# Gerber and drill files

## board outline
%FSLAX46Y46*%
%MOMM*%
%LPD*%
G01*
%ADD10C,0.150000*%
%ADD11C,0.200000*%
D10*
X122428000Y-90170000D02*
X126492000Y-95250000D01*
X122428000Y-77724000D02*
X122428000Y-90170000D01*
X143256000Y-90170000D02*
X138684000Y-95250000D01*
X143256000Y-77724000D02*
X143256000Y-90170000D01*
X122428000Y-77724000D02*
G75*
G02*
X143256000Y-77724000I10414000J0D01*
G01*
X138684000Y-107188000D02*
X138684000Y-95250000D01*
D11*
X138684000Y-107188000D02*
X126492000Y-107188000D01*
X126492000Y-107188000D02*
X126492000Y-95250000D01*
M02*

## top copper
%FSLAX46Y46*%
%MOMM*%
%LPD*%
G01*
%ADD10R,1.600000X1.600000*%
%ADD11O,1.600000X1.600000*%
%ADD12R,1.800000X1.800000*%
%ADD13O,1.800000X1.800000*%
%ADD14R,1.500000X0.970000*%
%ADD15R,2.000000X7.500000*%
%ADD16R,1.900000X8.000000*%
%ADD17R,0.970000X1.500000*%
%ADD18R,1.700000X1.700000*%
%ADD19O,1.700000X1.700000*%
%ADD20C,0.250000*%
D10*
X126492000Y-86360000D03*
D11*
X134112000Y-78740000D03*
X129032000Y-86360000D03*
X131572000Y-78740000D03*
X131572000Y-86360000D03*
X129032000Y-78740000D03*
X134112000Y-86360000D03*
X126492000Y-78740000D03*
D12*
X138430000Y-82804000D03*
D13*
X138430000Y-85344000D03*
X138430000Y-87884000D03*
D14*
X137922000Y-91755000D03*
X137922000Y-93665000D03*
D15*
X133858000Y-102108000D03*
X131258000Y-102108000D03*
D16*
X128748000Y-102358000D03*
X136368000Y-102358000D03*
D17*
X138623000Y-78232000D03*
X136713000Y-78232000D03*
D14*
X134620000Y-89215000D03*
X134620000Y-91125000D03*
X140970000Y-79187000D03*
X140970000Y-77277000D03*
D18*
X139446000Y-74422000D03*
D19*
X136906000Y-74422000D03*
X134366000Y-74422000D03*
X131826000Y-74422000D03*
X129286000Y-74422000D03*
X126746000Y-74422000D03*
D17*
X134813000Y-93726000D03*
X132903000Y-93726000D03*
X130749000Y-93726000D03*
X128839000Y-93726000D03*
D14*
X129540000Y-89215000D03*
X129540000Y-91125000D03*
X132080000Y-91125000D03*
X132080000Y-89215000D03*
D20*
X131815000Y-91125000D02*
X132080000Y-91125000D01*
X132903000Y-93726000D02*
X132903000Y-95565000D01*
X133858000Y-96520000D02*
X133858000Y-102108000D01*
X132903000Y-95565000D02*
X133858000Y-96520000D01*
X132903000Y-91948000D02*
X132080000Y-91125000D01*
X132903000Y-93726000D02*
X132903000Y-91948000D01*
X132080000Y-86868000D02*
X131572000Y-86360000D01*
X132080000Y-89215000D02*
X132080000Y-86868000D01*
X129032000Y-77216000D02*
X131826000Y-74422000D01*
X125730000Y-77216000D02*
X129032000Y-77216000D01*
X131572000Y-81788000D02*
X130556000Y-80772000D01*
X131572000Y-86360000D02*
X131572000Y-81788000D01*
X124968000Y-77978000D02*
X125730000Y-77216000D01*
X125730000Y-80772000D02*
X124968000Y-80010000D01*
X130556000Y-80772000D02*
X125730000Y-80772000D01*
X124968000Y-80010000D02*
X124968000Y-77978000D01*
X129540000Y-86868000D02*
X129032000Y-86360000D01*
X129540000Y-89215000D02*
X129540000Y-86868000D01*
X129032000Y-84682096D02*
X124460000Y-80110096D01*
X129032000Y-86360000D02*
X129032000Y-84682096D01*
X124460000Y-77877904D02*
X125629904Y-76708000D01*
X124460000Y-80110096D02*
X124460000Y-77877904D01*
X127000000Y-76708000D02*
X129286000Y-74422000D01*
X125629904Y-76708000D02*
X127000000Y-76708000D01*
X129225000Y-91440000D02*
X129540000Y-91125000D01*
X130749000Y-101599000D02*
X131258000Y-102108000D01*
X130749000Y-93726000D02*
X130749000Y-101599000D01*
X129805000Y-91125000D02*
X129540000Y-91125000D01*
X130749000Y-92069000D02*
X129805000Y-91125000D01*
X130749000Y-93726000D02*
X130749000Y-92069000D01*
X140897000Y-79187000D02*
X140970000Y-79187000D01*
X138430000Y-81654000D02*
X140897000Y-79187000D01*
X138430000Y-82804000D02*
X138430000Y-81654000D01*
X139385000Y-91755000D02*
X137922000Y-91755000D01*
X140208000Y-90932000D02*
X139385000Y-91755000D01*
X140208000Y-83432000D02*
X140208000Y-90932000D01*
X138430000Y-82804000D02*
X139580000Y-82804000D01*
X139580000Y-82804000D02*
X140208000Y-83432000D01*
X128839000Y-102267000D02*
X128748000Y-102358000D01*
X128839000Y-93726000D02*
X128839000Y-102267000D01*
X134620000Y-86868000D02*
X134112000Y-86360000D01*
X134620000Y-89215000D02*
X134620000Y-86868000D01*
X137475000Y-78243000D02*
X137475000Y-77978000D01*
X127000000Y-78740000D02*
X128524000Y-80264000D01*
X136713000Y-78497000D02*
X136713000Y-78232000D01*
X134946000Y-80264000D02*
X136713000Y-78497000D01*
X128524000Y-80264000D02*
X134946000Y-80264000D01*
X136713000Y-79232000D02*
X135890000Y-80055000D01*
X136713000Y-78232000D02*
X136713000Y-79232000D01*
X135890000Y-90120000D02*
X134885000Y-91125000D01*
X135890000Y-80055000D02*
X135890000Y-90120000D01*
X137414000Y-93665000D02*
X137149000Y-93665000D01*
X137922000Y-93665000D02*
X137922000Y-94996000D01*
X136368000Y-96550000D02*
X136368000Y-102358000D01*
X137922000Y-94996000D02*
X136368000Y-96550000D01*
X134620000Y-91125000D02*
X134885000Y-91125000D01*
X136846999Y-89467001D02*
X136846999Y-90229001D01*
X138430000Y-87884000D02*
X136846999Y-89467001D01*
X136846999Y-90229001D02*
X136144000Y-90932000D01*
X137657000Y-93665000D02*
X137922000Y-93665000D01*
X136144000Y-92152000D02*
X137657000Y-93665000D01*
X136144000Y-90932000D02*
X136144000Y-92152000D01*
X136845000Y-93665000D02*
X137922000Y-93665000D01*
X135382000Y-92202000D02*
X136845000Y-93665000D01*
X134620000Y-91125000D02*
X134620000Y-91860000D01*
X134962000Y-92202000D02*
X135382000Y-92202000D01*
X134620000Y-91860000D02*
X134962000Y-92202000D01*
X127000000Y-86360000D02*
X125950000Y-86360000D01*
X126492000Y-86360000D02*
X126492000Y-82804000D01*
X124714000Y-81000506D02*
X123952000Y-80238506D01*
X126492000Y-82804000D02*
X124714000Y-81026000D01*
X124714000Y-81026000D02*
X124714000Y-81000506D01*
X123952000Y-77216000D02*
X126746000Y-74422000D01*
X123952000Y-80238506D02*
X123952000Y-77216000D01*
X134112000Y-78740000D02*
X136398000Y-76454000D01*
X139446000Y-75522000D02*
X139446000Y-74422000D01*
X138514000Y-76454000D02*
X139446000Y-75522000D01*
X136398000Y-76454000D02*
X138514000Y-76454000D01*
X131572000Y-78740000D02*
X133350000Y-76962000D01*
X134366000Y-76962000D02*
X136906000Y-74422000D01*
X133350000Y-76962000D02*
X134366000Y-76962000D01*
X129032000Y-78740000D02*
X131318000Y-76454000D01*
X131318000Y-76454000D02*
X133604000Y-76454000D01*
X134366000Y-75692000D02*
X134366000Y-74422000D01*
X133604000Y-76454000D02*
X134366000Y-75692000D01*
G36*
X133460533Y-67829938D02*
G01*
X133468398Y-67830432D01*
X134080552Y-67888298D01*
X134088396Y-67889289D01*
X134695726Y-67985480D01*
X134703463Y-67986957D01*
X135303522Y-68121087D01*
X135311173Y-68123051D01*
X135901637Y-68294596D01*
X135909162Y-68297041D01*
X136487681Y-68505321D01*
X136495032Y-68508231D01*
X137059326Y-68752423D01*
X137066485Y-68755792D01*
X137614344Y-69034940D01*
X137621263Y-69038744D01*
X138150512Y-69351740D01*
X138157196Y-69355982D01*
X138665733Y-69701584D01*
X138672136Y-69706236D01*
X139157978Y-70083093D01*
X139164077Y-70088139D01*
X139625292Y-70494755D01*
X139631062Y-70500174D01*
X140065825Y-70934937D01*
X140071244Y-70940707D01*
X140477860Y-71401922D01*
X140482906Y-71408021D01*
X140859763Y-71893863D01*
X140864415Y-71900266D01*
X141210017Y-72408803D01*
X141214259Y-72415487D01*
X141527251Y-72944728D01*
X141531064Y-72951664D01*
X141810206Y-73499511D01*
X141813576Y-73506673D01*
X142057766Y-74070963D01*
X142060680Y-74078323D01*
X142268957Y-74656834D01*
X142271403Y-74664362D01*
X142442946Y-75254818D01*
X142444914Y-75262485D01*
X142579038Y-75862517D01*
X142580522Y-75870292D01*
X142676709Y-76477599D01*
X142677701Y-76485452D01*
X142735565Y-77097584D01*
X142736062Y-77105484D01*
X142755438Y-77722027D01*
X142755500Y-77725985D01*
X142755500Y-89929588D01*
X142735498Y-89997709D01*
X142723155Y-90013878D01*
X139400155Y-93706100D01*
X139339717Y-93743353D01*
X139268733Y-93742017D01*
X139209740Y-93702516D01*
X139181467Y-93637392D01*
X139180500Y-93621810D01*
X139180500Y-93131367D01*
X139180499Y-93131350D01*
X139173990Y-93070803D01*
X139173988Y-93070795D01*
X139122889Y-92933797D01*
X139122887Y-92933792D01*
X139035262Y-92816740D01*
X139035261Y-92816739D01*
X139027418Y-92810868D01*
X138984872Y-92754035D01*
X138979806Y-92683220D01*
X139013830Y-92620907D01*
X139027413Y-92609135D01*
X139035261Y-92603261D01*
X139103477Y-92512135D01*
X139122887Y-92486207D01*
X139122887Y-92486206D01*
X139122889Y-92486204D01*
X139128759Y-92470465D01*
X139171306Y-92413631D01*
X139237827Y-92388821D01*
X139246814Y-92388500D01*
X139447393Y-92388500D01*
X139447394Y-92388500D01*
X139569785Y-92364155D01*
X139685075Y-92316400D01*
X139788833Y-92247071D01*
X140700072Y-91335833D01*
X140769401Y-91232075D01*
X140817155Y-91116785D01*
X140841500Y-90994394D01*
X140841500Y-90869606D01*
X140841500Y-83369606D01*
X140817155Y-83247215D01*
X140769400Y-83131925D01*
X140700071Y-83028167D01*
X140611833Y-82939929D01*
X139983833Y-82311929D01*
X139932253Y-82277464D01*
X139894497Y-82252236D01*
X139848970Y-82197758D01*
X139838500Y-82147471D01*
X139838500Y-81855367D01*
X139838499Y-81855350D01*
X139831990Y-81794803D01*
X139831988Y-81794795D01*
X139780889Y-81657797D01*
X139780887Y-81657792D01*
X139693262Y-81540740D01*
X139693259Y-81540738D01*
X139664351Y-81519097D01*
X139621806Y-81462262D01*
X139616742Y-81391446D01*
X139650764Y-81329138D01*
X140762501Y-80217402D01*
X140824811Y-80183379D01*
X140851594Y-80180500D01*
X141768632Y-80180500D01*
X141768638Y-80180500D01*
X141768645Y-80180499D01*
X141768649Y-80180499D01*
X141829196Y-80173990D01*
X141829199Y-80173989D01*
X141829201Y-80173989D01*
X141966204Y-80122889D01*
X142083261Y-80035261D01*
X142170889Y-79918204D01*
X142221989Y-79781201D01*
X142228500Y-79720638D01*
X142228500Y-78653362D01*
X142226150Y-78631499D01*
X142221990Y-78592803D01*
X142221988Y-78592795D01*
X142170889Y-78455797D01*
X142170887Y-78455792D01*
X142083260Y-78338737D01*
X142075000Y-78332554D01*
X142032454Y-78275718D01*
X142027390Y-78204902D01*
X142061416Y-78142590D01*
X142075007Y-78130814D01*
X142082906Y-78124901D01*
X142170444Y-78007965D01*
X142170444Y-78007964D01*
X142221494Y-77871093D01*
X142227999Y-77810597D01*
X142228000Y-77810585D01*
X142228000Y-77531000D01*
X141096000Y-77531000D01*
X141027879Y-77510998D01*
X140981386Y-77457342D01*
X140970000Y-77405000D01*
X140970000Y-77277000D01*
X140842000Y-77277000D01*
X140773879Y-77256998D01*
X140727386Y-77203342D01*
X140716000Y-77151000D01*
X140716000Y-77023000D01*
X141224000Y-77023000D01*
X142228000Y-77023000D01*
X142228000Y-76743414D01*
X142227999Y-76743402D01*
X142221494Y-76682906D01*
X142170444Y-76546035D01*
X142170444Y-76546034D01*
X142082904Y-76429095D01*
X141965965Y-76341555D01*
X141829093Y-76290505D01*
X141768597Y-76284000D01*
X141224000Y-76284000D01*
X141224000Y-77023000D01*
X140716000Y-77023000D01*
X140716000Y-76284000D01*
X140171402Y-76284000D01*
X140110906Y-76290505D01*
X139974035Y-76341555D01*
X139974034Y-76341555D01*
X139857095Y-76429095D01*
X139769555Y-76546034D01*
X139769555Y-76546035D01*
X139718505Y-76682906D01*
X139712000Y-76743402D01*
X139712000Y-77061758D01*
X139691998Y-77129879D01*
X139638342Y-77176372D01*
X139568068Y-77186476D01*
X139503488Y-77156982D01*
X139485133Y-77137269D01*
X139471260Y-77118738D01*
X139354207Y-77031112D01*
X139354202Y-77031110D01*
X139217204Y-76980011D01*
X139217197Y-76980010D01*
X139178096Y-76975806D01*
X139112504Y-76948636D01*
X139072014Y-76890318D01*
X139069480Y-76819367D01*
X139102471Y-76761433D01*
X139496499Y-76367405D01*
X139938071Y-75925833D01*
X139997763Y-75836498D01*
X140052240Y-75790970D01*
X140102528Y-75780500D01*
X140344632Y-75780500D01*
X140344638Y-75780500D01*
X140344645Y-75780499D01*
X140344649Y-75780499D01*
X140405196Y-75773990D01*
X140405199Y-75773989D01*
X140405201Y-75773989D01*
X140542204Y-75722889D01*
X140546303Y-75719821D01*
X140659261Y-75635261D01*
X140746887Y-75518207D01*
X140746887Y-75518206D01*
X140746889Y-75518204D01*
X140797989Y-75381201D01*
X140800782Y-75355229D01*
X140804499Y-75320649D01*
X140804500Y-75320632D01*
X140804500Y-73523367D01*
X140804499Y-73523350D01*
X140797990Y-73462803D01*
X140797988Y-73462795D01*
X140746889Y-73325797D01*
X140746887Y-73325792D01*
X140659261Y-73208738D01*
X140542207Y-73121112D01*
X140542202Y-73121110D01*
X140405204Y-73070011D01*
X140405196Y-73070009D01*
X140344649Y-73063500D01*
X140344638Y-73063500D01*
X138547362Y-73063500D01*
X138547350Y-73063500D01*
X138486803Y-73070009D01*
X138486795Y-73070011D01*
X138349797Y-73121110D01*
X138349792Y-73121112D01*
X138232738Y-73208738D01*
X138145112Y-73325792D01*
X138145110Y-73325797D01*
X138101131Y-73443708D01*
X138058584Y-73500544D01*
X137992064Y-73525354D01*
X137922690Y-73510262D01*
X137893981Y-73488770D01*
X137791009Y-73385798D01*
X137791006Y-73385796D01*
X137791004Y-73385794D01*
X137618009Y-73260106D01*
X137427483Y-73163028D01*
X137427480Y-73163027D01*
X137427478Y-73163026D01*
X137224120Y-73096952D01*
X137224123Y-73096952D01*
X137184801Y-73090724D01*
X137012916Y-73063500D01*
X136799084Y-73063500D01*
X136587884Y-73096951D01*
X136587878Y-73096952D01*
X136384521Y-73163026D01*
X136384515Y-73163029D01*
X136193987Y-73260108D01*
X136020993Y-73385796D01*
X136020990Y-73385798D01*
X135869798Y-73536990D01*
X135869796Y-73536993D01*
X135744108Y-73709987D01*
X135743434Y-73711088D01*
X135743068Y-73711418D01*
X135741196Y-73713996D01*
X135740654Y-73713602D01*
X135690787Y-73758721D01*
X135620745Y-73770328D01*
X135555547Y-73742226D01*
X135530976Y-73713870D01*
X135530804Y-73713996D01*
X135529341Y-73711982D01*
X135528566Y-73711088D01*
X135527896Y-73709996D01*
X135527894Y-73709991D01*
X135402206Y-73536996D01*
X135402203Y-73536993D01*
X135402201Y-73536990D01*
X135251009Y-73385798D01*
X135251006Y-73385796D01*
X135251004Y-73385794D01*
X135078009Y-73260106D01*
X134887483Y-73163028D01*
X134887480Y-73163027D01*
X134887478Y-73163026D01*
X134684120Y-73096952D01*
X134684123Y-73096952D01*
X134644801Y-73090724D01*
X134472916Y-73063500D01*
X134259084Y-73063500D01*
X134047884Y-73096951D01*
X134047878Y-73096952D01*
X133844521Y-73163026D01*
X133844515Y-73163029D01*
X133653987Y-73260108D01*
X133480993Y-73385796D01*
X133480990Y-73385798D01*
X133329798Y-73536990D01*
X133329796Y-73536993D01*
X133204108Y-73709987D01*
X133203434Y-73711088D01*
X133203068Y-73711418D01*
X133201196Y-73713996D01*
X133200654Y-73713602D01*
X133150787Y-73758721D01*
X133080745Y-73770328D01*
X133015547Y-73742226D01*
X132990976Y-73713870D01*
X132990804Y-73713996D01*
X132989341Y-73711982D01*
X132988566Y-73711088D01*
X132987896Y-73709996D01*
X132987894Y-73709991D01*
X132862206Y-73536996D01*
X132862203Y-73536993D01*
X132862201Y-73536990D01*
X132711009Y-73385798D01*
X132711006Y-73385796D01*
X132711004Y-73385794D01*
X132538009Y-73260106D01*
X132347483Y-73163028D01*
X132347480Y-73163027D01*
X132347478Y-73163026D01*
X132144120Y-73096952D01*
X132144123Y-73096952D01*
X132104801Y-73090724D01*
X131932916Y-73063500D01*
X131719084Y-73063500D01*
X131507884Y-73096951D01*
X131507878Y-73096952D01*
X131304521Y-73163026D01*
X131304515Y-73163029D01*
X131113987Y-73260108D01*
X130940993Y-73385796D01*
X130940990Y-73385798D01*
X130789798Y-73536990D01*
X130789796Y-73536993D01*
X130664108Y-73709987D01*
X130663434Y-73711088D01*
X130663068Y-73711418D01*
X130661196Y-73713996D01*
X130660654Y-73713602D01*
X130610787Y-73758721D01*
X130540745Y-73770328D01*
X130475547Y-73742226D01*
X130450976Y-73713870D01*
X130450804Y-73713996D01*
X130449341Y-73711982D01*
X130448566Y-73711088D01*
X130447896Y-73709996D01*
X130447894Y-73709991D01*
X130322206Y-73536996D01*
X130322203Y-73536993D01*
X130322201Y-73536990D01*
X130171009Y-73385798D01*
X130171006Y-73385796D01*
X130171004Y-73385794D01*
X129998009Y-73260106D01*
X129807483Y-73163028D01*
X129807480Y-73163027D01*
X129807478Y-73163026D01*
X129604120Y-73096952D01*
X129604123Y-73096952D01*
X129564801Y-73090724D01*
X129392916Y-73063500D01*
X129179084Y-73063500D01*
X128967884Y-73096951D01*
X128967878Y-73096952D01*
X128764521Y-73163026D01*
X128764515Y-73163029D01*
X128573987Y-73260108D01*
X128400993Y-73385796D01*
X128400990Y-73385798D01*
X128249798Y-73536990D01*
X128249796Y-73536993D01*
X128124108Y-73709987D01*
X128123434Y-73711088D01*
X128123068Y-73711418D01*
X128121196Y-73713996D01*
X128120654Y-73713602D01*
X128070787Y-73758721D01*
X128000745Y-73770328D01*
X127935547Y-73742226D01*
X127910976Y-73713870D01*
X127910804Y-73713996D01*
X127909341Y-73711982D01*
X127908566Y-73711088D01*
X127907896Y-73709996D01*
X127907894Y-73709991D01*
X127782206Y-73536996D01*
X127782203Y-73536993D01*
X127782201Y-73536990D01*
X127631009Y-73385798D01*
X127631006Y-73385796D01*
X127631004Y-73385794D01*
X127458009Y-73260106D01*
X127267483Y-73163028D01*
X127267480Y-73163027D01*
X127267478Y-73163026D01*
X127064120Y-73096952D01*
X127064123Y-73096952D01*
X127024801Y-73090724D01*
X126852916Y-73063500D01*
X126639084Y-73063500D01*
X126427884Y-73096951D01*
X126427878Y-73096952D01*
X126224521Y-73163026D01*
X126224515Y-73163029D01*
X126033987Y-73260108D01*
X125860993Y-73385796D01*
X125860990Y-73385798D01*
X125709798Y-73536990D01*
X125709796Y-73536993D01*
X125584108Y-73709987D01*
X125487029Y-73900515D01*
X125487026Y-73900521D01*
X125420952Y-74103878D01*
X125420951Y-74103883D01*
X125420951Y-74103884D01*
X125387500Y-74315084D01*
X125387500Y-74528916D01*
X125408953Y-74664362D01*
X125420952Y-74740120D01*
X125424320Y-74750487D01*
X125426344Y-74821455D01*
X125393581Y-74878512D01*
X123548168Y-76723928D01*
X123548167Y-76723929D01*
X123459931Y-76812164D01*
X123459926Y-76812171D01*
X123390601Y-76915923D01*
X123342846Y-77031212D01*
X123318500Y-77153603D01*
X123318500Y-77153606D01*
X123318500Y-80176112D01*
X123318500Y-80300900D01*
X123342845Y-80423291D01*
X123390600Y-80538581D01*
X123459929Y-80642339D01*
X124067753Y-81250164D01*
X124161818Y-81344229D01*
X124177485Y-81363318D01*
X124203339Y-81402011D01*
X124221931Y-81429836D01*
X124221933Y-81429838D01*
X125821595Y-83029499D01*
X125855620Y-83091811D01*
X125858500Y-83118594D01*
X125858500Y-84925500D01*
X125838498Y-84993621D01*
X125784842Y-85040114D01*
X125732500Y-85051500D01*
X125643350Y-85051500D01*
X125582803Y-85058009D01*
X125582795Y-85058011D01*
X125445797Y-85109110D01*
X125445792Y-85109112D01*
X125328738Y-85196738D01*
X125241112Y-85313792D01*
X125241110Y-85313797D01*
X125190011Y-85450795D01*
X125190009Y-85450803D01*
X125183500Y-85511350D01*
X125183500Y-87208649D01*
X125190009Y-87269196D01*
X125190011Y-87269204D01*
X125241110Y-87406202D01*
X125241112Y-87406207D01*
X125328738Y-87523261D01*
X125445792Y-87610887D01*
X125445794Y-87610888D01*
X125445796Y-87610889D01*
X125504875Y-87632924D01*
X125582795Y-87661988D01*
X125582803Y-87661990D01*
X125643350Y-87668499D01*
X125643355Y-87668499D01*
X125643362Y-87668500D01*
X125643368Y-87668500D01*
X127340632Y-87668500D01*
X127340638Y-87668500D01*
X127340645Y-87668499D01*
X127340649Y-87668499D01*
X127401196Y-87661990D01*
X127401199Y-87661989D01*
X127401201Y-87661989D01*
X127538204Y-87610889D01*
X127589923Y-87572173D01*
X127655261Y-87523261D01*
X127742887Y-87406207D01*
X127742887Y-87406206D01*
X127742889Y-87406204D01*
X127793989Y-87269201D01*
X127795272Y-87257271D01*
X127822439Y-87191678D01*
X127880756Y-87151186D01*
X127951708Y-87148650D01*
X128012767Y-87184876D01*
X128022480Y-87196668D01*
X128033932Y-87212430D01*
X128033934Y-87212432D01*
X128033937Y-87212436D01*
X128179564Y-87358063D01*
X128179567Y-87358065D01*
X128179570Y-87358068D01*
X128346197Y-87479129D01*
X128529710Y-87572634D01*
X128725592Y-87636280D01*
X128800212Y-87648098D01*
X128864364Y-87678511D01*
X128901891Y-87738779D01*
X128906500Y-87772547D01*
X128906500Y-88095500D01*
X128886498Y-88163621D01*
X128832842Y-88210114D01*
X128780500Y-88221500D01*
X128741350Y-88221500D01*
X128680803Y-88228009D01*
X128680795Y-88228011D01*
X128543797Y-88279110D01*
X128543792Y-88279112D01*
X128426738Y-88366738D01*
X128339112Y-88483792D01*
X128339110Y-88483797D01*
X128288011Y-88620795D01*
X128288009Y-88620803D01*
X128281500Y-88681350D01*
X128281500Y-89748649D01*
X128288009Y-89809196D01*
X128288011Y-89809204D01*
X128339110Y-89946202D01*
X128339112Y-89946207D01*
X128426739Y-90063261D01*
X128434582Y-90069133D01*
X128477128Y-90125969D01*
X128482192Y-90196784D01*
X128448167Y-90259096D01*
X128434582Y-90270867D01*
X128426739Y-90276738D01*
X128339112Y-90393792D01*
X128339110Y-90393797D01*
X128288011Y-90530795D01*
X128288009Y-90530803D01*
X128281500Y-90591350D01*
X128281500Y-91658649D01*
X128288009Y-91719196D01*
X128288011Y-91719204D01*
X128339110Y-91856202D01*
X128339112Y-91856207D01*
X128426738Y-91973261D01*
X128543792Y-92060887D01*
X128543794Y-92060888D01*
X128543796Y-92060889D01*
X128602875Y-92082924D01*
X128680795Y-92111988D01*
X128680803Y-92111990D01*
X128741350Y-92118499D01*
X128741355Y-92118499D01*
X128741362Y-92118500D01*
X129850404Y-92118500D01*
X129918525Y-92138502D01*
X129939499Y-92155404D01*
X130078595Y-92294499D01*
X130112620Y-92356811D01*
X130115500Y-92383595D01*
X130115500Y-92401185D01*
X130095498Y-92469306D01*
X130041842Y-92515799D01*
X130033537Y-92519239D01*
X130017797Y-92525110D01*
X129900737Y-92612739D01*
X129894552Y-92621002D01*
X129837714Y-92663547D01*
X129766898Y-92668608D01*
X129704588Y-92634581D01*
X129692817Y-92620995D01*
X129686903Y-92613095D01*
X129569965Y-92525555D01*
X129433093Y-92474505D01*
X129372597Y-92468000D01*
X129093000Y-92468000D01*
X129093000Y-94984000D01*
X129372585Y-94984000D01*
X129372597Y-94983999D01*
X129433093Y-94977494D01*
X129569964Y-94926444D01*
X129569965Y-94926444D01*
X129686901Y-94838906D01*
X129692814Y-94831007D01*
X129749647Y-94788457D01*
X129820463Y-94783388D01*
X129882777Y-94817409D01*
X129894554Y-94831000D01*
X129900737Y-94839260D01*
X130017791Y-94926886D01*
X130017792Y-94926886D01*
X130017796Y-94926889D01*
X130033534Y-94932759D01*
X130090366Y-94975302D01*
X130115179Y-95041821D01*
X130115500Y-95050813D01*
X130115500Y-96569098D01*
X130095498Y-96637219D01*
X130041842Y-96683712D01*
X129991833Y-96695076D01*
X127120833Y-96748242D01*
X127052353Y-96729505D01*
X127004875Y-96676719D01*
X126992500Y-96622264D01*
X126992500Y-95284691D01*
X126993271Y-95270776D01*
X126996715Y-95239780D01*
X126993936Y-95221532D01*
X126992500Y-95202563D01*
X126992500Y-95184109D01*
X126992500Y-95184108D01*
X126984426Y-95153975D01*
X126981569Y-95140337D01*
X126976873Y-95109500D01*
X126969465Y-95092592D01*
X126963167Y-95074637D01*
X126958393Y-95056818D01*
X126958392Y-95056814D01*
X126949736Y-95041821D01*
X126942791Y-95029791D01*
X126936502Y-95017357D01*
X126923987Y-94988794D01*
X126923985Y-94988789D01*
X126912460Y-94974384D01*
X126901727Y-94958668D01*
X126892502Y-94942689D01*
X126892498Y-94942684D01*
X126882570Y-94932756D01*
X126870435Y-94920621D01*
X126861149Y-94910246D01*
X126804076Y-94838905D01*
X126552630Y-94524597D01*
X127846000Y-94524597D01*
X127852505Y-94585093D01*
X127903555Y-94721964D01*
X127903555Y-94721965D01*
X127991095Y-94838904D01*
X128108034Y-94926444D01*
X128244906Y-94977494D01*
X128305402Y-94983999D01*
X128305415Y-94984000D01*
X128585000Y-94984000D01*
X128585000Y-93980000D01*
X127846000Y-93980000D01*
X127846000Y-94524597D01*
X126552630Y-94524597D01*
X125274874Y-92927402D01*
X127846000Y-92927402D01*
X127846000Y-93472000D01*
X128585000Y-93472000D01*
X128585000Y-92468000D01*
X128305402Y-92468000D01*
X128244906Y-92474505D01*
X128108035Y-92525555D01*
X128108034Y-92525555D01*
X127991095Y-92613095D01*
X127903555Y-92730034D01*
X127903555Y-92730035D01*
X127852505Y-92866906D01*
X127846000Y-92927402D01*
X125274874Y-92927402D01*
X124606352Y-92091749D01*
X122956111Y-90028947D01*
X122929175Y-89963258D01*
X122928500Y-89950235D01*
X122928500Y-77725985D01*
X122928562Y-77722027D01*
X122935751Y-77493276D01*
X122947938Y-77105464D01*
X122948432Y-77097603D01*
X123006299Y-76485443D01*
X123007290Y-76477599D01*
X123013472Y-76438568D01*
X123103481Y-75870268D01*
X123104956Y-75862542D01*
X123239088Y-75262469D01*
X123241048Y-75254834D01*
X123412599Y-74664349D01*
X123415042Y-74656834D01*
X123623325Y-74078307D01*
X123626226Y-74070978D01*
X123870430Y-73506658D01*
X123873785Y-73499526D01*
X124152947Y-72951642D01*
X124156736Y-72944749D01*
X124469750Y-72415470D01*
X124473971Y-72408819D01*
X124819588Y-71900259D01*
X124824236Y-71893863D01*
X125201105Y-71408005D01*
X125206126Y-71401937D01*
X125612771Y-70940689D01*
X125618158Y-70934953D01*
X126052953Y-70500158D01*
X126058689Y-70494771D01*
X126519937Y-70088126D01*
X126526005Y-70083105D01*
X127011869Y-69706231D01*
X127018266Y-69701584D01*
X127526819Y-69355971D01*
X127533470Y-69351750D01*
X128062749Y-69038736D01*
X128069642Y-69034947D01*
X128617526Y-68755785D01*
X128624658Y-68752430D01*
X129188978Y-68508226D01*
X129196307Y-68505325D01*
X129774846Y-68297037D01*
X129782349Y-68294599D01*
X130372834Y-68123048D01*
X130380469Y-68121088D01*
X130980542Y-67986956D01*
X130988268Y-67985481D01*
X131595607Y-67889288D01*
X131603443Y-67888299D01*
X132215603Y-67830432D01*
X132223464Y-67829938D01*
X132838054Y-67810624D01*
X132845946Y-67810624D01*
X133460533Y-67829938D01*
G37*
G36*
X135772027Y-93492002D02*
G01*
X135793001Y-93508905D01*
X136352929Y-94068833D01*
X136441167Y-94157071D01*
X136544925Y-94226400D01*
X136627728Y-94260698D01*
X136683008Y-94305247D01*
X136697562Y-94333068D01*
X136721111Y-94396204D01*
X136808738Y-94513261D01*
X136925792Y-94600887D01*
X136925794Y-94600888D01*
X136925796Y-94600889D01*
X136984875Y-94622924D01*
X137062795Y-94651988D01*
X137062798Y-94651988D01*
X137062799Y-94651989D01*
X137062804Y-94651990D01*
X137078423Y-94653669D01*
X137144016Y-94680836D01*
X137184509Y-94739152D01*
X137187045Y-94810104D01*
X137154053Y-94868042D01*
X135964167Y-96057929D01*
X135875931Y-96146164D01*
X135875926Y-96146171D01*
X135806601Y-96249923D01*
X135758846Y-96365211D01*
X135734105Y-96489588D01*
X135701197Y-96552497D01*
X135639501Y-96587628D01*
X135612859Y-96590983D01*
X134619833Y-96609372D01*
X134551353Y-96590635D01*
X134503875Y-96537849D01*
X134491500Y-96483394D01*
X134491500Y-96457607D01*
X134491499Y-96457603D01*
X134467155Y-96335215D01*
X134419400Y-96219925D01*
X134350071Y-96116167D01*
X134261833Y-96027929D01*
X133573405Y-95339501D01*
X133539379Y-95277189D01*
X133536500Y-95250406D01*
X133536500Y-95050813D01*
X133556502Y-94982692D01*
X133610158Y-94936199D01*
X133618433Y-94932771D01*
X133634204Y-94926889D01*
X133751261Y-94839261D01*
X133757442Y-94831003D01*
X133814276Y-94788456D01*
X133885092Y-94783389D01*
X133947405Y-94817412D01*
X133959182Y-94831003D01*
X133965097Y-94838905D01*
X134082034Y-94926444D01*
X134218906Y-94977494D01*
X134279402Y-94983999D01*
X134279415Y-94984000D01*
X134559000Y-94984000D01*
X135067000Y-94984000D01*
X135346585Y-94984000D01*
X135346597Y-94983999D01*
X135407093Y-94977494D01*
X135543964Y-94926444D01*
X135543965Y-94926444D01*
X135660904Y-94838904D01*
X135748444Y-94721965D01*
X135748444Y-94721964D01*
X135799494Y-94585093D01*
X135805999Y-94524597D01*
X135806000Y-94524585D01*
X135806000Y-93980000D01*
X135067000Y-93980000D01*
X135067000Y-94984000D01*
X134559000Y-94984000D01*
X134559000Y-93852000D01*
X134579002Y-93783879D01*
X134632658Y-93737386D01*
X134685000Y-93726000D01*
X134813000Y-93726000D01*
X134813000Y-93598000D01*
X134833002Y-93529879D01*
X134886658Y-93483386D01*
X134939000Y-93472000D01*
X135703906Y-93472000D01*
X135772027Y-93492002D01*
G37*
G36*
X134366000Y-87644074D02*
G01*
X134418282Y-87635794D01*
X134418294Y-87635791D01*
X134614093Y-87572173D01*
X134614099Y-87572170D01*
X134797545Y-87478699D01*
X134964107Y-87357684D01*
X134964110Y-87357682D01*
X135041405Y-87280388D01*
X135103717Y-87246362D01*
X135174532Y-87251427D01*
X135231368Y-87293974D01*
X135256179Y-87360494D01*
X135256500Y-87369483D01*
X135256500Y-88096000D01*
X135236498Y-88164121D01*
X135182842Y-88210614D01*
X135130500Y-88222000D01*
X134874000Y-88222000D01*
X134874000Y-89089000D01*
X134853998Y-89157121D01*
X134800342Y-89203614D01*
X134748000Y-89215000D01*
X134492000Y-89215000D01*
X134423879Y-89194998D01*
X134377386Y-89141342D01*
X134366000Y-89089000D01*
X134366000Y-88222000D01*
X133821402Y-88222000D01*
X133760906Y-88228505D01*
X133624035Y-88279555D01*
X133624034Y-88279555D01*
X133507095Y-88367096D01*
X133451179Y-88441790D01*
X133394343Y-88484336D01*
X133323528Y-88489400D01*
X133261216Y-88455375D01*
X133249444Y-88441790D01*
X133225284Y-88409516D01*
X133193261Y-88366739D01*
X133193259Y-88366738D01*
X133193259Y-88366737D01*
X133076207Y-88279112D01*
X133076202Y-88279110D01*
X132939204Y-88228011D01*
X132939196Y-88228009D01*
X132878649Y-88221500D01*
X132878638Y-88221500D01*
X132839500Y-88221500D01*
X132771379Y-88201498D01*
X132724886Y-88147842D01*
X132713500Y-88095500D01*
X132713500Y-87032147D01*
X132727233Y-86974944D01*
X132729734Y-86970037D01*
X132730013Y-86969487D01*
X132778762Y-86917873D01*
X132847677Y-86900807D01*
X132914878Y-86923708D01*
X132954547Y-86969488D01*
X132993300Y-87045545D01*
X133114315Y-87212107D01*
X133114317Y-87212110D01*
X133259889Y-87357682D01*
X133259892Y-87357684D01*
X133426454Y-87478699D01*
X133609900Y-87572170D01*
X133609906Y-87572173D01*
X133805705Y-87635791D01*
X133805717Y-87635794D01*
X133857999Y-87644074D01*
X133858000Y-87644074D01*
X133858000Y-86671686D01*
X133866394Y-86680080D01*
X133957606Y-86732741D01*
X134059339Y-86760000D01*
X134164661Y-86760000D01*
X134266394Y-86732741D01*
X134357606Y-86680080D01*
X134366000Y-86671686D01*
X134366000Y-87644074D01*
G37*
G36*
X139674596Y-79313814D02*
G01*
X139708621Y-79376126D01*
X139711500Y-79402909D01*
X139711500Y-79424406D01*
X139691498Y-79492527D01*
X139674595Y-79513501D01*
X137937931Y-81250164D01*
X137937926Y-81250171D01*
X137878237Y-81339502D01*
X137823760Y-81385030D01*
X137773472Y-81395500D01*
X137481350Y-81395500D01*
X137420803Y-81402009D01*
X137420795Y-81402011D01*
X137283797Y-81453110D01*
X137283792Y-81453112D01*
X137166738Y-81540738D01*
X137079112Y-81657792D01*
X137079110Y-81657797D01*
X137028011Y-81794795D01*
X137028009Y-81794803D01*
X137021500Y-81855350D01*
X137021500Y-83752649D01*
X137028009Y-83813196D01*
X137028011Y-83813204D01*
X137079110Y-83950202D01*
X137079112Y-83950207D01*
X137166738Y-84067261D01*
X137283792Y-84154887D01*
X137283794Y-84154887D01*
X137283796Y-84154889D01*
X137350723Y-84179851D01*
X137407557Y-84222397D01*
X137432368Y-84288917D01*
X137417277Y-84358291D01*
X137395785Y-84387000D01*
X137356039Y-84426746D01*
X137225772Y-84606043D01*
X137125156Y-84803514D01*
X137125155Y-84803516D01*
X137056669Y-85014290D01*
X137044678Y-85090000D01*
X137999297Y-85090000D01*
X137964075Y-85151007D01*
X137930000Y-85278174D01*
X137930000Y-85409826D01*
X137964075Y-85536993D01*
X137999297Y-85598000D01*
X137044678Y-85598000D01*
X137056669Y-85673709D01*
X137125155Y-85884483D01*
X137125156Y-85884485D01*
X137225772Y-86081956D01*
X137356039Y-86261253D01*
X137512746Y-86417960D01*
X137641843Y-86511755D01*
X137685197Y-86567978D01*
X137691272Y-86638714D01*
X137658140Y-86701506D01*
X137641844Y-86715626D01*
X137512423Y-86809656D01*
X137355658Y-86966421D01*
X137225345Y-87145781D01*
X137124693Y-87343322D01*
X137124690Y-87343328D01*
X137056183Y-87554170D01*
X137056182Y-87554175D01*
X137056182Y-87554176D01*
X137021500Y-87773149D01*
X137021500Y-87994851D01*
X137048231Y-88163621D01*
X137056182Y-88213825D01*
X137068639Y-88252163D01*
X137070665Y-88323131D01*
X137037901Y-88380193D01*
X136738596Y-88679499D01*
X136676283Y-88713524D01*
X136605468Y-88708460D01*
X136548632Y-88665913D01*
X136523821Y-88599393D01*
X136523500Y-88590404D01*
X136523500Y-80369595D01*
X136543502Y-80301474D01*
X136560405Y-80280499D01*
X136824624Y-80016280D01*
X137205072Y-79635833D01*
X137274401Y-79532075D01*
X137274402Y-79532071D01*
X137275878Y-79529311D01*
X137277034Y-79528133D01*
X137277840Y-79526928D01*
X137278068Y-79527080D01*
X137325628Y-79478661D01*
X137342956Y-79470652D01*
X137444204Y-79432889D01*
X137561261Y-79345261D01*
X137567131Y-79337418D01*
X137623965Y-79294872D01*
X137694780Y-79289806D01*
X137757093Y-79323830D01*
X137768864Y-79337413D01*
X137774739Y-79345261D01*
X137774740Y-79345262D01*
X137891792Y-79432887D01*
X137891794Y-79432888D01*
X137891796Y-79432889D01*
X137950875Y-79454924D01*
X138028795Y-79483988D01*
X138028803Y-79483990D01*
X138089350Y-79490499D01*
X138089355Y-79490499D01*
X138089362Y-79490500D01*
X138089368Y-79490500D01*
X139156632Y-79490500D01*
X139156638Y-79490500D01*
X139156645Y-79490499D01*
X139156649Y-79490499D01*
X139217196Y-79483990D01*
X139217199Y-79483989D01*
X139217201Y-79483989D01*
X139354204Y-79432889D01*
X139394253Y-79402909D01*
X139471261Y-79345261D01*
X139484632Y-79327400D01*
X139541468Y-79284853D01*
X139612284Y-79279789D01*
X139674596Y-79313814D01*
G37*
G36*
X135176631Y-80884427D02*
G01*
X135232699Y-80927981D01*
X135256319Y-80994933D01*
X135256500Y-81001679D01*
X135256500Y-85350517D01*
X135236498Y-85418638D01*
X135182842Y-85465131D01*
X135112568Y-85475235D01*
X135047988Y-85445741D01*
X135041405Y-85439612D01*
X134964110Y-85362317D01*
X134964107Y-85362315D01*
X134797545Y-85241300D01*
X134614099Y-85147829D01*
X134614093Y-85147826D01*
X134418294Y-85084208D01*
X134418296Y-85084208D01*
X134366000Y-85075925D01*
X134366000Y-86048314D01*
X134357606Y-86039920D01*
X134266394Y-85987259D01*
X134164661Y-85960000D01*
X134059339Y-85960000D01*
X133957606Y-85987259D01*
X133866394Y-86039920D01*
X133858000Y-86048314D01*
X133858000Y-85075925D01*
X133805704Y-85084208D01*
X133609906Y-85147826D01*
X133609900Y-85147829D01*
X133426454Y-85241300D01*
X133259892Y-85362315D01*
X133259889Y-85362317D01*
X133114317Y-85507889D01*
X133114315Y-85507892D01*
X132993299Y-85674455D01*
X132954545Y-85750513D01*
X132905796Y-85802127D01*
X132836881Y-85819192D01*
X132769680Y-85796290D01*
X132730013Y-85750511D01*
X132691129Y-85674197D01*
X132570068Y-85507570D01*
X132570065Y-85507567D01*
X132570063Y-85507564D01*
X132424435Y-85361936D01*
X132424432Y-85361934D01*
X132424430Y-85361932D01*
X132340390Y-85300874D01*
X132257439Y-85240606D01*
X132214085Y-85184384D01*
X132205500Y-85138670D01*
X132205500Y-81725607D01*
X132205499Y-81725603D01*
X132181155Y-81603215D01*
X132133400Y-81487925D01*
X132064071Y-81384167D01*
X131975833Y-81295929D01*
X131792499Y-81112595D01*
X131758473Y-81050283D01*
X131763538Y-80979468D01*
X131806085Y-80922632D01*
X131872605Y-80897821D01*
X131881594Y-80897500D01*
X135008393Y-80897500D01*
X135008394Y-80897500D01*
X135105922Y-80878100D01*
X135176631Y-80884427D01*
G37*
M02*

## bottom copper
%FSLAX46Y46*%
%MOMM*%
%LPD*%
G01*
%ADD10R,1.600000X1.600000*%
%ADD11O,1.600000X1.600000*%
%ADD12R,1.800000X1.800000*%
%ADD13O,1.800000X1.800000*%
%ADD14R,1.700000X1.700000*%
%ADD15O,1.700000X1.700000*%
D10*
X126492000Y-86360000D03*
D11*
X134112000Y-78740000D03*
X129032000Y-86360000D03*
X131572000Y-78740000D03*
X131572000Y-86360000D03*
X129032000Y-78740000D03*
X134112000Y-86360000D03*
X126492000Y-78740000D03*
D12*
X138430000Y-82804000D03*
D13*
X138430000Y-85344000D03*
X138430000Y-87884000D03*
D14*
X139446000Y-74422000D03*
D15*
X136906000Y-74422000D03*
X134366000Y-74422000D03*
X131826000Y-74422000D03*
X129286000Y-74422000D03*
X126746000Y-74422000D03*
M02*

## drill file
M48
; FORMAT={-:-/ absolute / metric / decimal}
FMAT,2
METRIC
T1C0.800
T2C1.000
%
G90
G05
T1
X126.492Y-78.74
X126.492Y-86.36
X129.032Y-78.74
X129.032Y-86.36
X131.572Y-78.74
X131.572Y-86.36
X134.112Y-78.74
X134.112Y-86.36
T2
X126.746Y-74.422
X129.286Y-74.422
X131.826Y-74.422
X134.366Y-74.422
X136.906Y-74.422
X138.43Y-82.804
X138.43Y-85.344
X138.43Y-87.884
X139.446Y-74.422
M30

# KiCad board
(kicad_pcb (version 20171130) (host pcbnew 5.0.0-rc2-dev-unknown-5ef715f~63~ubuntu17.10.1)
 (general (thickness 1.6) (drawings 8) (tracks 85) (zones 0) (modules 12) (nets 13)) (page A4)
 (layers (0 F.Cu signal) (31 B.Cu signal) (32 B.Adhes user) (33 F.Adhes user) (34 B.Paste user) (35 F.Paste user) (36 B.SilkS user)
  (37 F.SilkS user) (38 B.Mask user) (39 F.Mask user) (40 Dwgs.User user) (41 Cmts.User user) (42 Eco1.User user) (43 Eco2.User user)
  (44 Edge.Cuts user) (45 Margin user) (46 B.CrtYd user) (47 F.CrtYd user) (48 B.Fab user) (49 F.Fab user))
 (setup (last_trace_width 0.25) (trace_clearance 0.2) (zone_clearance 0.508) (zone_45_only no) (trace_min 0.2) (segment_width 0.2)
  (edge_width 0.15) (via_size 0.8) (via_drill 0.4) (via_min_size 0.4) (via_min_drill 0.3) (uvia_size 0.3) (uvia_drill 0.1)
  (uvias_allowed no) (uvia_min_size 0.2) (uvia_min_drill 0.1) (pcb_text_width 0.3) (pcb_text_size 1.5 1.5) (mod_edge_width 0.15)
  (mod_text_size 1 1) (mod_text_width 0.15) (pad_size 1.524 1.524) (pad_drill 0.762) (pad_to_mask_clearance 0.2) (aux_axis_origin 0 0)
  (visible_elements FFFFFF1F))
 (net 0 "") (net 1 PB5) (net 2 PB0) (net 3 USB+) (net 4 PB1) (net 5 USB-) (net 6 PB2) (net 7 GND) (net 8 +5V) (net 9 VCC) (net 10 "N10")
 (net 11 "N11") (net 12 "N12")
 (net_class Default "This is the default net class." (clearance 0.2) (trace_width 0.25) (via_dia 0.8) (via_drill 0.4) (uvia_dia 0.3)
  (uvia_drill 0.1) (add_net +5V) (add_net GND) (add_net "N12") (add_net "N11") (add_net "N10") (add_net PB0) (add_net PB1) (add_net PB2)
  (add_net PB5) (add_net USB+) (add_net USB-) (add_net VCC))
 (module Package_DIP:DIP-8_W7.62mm (layer F.Cu) (at 126.492 86.36 90)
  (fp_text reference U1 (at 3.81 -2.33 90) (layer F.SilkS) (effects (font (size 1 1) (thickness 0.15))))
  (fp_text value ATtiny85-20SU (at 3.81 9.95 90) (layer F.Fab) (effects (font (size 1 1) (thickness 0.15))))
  (pad 1 thru_hole rect (at 0 0 90) (size 1.6 1.6) (drill 0.8) (layers *.Cu *.Mask) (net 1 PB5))
  (pad 5 thru_hole oval (at 7.62 7.62 90) (size 1.6 1.6) (drill 0.8) (layers *.Cu *.Mask) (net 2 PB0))
  (pad 2 thru_hole oval (at 0 2.54 90) (size 1.6 1.6) (drill 0.8) (layers *.Cu *.Mask) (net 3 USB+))
  (pad 6 thru_hole oval (at 7.62 5.08 90) (size 1.6 1.6) (drill 0.8) (layers *.Cu *.Mask) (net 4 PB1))
  (pad 3 thru_hole oval (at 0 5.08 90) (size 1.6 1.6) (drill 0.8) (layers *.Cu *.Mask) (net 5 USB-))
  (pad 7 thru_hole oval (at 7.62 2.54 90) (size 1.6 1.6) (drill 0.8) (layers *.Cu *.Mask) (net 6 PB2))
  (pad 4 thru_hole oval (at 0 7.62 90) (size 1.6 1.6) (drill 0.8) (layers *.Cu *.Mask) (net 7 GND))
  (pad 8 thru_hole oval (at 7.62 0 90) (size 1.6 1.6) (drill 0.8) (layers *.Cu *.Mask) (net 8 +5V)))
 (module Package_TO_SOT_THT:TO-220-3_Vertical (layer F.Cu) (at 138.43 82.804 270)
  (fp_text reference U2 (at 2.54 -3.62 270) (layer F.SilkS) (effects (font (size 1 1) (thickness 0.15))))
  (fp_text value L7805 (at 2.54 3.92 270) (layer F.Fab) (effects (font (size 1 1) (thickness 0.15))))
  (pad 1 thru_hole rect (at 0 0 270) (size 1.8 1.8) (drill 1) (layers *.Cu *.Mask) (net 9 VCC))
  (pad 2 thru_hole oval (at 2.54 0 270) (size 1.8 1.8) (drill 1) (layers *.Cu *.Mask) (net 7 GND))
  (pad 3 thru_hole oval (at 5.08 0 270) (size 1.8 1.8) (drill 1) (layers *.Cu *.Mask) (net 8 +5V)))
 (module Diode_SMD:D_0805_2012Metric (layer F.Cu) (at 137.922 92.71 270)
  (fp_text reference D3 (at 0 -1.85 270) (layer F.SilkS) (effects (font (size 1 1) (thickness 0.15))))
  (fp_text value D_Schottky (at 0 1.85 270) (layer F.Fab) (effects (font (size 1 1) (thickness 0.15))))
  (pad 1 smd rect (at -0.955 0 270) (size 0.97 1.5) (layers F.Cu F.Paste F.Mask) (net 9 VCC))
  (pad 2 smd rect (at 0.955 0 270) (size 0.97 1.5) (layers F.Cu F.Paste F.Mask) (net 8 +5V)))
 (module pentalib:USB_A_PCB (layer F.Cu) (at 132.558 107.258)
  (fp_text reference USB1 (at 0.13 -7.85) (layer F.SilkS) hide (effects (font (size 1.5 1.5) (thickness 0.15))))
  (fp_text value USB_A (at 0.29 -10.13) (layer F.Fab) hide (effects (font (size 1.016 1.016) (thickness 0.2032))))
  (pad 2 connect rect (at 1.3 -5.15) (size 2 7.5) (layers F.Cu F.Mask) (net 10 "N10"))
  (pad 3 connect rect (at -1.3 -5.15) (size 2 7.5) (layers F.Cu F.Mask) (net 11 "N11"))
  (pad 4 connect rect (at -3.81 -4.9) (size 1.9 8) (layers F.Cu F.Mask) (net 7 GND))
  (pad 1 connect rect (at 3.81 -4.9) (size 1.9 8) (layers F.Cu F.Mask) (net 8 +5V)))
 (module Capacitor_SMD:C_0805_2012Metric (layer F.Cu) (at 137.668 78.232 180)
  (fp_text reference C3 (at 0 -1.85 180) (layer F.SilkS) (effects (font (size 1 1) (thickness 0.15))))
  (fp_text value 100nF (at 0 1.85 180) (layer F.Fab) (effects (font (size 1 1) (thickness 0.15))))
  (pad 1 smd rect (at -0.955 0 180) (size 0.97 1.5) (layers F.Cu F.Paste F.Mask) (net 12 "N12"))
  (pad 2 smd rect (at 0.955 0 180) (size 0.97 1.5) (layers F.Cu F.Paste F.Mask) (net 8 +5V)))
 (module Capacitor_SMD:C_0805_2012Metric (layer F.Cu) (at 134.62 90.17 90)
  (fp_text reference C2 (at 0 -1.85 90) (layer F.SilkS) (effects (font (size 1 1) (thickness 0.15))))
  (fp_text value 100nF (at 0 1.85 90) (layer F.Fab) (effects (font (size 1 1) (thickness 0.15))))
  (pad 2 smd rect (at 0.955 0 90) (size 0.97 1.5) (layers F.Cu F.Paste F.Mask) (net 7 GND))
  (pad 1 smd rect (at -0.955 0 90) (size 0.97 1.5) (layers F.Cu F.Paste F.Mask) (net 8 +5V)))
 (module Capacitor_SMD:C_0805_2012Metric (layer F.Cu) (at 140.97 78.232 90)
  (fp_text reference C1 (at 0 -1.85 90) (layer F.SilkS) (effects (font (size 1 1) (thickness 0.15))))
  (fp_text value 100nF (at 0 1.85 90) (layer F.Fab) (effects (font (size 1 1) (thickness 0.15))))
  (pad 1 smd rect (at -0.955 0 90) (size 0.97 1.5) (layers F.Cu F.Paste F.Mask) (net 9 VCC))
  (pad 2 smd rect (at 0.955 0 90) (size 0.97 1.5) (layers F.Cu F.Paste F.Mask) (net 7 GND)))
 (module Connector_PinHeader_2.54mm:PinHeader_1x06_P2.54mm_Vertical (layer F.Cu) (at 139.446 74.422 270)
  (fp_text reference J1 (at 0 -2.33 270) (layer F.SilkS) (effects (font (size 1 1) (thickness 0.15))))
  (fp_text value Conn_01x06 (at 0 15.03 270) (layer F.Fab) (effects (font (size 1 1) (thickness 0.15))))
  (pad 1 thru_hole rect (at 0 0 270) (size 1.7 1.7) (drill 1) (layers *.Cu *.Mask) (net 2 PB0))
  (pad 2 thru_hole oval (at 0 2.54 270) (size 1.7 1.7) (drill 1) (layers *.Cu *.Mask) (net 4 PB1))
  (pad 3 thru_hole oval (at 0 5.08 270) (size 1.7 1.7) (drill 1) (layers *.Cu *.Mask) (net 6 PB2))
  (pad 4 thru_hole oval (at 0 7.62 270) (size 1.7 1.7) (drill 1) (layers *.Cu *.Mask) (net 5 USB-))
  (pad 5 thru_hole oval (at 0 10.16 270) (size 1.7 1.7) (drill 1) (layers *.Cu *.Mask) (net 3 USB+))
  (pad 6 thru_hole oval (at 0 12.7 270) (size 1.7 1.7) (drill 1) (layers *.Cu *.Mask) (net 1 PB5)))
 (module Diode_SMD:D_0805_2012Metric (layer F.Cu) (at 133.858 93.726)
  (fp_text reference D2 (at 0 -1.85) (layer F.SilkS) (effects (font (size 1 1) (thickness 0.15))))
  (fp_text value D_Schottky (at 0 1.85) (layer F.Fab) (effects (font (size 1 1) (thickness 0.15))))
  (pad 2 smd rect (at 0.955 0) (size 0.97 1.5) (layers F.Cu F.Paste F.Mask) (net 7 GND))
  (pad 1 smd rect (at -0.955 0) (size 0.97 1.5) (layers F.Cu F.Paste F.Mask) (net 10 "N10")))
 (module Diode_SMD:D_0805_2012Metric (layer F.Cu) (at 129.794 93.726 180)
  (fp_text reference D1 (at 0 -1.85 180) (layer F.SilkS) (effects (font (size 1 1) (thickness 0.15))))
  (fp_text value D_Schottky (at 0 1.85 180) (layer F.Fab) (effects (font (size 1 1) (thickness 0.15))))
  (pad 1 smd rect (at -0.955 0 180) (size 0.97 1.5) (layers F.Cu F.Paste F.Mask) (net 11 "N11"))
  (pad 2 smd rect (at 0.955 0 180) (size 0.97 1.5) (layers F.Cu F.Paste F.Mask) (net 7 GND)))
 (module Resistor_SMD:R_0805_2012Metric (layer F.Cu) (at 129.54 90.17 90)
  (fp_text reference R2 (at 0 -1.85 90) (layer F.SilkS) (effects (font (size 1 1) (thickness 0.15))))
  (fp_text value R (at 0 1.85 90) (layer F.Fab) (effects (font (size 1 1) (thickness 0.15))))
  (pad 2 smd rect (at 0.955 0 90) (size 0.97 1.5) (layers F.Cu F.Paste F.Mask) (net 3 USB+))
  (pad 1 smd rect (at -0.955 0 90) (size 0.97 1.5) (layers F.Cu F.Paste F.Mask) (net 11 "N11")))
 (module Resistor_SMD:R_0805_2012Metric (layer F.Cu) (at 132.08 90.17 90)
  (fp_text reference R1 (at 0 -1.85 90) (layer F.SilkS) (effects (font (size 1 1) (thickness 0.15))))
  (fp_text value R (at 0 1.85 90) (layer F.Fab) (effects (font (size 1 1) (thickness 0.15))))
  (pad 1 smd rect (at -0.955 0 90) (size 0.97 1.5) (layers F.Cu F.Paste F.Mask) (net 10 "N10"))
  (pad 2 smd rect (at 0.955 0 90) (size 0.97 1.5) (layers F.Cu F.Paste F.Mask) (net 5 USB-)))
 (gr_line (start 122.428 90.17) (end 126.492 95.25) (layer Edge.Cuts) (width 0.15))
 (gr_line (start 122.428 77.724) (end 122.428 90.17) (layer Edge.Cuts) (width 0.15))
 (gr_line (start 143.256 90.17) (end 138.684 95.25) (layer Edge.Cuts) (width 0.15))
 (gr_line (start 143.256 77.724) (end 143.256 90.17) (layer Edge.Cuts) (width 0.15))
 (gr_arc (start 132.842 77.724) (end 143.256 77.724) (angle -180) (layer Edge.Cuts) (width 0.15))
 (gr_line (start 138.684 107.188) (end 138.684 95.25) (layer Edge.Cuts) (width 0.15))
 (gr_line (start 138.684 107.188) (end 126.492 107.188) (layer Edge.Cuts) (width 0.2))
 (gr_line (start 126.492 107.188) (end 126.492 95.25) (layer Edge.Cuts) (width 0.2))
 (segment (start 131.815 91.125) (end 132.08 91.125) (width 0.25) (layer F.Cu) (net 10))
 (segment (start 132.903 93.726) (end 132.903 95.565) (width 0.25) (layer F.Cu) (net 10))
 (segment (start 133.858 96.52) (end 133.858 102.108) (width 0.25) (layer F.Cu) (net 10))
 (segment (start 132.903 95.565) (end 133.858 96.52) (width 0.25) (layer F.Cu) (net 10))
 (segment (start 132.903 91.948) (end 132.08 91.125) (width 0.25) (layer F.Cu) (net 10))
 (segment (start 132.903 93.726) (end 132.903 91.948) (width 0.25) (layer F.Cu) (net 10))
 (segment (start 132.08 86.868) (end 131.572 86.36) (width 0.25) (layer F.Cu) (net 5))
 (segment (start 132.08 89.215) (end 132.08 86.868) (width 0.25) (layer F.Cu) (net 5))
 (segment (start 129.032 77.216) (end 131.826 74.422) (width 0.25) (layer F.Cu) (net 5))
 (segment (start 125.73 77.216) (end 129.032 77.216) (width 0.25) (layer F.Cu) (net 5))
 (segment (start 131.572 81.788) (end 130.556 80.772) (width 0.25) (layer F.Cu) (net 5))
 (segment (start 131.572 86.36) (end 131.572 81.788) (width 0.25) (layer F.Cu) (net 5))
 (segment (start 124.968 77.978) (end 125.73 77.216) (width 0.25) (layer F.Cu) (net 5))
 (segment (start 125.73 80.772) (end 124.968 80.01) (width 0.25) (layer F.Cu) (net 5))
 (segment (start 130.556 80.772) (end 125.73 80.772) (width 0.25) (layer F.Cu) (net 5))
 (segment (start 124.968 80.01) (end 124.968 77.978) (width 0.25) (layer F.Cu) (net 5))
 (segment (start 129.54 86.868) (end 129.032 86.36) (width 0.25) (layer F.Cu) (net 3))
 (segment (start 129.54 89.215) (end 129.54 86.868) (width 0.25) (layer F.Cu) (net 3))
 (segment (start 129.032 84.682096) (end 124.46 80.110096) (width 0.25) (layer F.Cu) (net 3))
 (segment (start 129.032 86.36) (end 129.032 84.682096) (width 0.25) (layer F.Cu) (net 3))
 (segment (start 124.46 77.877904) (end 125.629904 76.708) (width 0.25) (layer F.Cu) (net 3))
 (segment (start 124.46 80.110096) (end 124.46 77.877904) (width 0.25) (layer F.Cu) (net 3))
 (segment (start 127 76.708) (end 129.286 74.422) (width 0.25) (layer F.Cu) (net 3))
 (segment (start 125.629904 76.708) (end 127 76.708) (width 0.25) (layer F.Cu) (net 3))
 (segment (start 129.225 91.44) (end 129.54 91.125) (width 0.25) (layer F.Cu) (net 11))
 (segment (start 130.749 101.599) (end 131.258 102.108) (width 0.25) (layer F.Cu) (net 11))
 (segment (start 130.749 93.726) (end 130.749 101.599) (width 0.25) (layer F.Cu) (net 11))
 (segment (start 129.805 91.125) (end 129.54 91.125) (width 0.25) (layer F.Cu) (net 11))
 (segment (start 130.749 92.069) (end 129.805 91.125) (width 0.25) (layer F.Cu) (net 11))
 (segment (start 130.749 93.726) (end 130.749 92.069) (width 0.25) (layer F.Cu) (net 11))
 (segment (start 140.897 79.187) (end 140.97 79.187) (width 0.25) (layer F.Cu) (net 9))
 (segment (start 138.43 81.654) (end 140.897 79.187) (width 0.25) (layer F.Cu) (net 9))
 (segment (start 138.43 82.804) (end 138.43 81.654) (width 0.25) (layer F.Cu) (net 9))
 (segment (start 139.385 91.755) (end 137.922 91.755) (width 0.25) (layer F.Cu) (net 9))
 (segment (start 140.208 90.932) (end 139.385 91.755) (width 0.25) (layer F.Cu) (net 9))
 (segment (start 140.208 83.432) (end 140.208 90.932) (width 0.25) (layer F.Cu) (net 9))
 (segment (start 138.43 82.804) (end 139.58 82.804) (width 0.25) (layer F.Cu) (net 9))
 (segment (start 139.58 82.804) (end 140.208 83.432) (width 0.25) (layer F.Cu) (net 9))
 (segment (start 128.839 102.267) (end 128.748 102.358) (width 0.25) (layer F.Cu) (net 7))
 (segment (start 128.839 93.726) (end 128.839 102.267) (width 0.25) (layer F.Cu) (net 7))
 (segment (start 134.62 86.868) (end 134.112 86.36) (width 0.25) (layer F.Cu) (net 7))
 (segment (start 134.62 89.215) (end 134.62 86.868) (width 0.25) (layer F.Cu) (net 7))
 (segment (start 137.475 78.243) (end 137.475 77.978) (width 0.25) (layer F.Cu) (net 8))
 (segment (start 127 78.74) (end 128.524 80.264) (width 0.25) (layer F.Cu) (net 8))
 (segment (start 136.713 78.497) (end 136.713 78.232) (width 0.25) (layer F.Cu) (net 8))
 (segment (start 134.946 80.264) (end 136.713 78.497) (width 0.25) (layer F.Cu) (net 8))
 (segment (start 128.524 80.264) (end 134.946 80.264) (width 0.25) (layer F.Cu) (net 8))
 (segment (start 136.713 79.232) (end 135.89 80.055) (width 0.25) (layer F.Cu) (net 8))
 (segment (start 136.713 78.232) (end 136.713 79.232) (width 0.25) (layer F.Cu) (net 8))
 (segment (start 135.89 90.12) (end 134.885 91.125) (width 0.25) (layer F.Cu) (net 8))
 (segment (start 135.89 80.055) (end 135.89 90.12) (width 0.25) (layer F.Cu) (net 8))
 (segment (start 137.414 93.665) (end 137.149 93.665) (width 0.25) (layer F.Cu) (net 8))
 (segment (start 137.922 93.665) (end 137.922 94.996) (width 0.25) (layer F.Cu) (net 8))
 (segment (start 136.368 96.55) (end 136.368 102.358) (width 0.25) (layer F.Cu) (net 8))
 (segment (start 137.922 94.996) (end 136.368 96.55) (width 0.25) (layer F.Cu) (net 8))
 (segment (start 134.62 91.125) (end 134.885 91.125) (width 0.25) (layer F.Cu) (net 8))
 (segment (start 136.846999 89.467001) (end 136.846999 90.229001) (width 0.25) (layer F.Cu) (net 8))
 (segment (start 138.43 87.884) (end 136.846999 89.467001) (width 0.25) (layer F.Cu) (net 8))
 (segment (start 136.846999 90.229001) (end 136.144 90.932) (width 0.25) (layer F.Cu) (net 8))
 (segment (start 137.657 93.665) (end 137.922 93.665) (width 0.25) (layer F.Cu) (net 8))
 (segment (start 136.144 92.152) (end 137.657 93.665) (width 0.25) (layer F.Cu) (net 8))
 (segment (start 136.144 90.932) (end 136.144 92.152) (width 0.25) (layer F.Cu) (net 8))
 (segment (start 136.845 93.665) (end 137.922 93.665) (width 0.25) (layer F.Cu) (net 8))
 (segment (start 135.382 92.202) (end 136.845 93.665) (width 0.25) (layer F.Cu) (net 8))
 (segment (start 134.62 91.125) (end 134.62 91.86) (width 0.25) (layer F.Cu) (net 8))
 (segment (start 134.962 92.202) (end 135.382 92.202) (width 0.25) (layer F.Cu) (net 8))
 (segment (start 134.62 91.86) (end 134.962 92.202) (width 0.25) (layer F.Cu) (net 8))
 (segment (start 127 86.36) (end 125.95 86.36) (width 0.25) (layer F.Cu) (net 1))
 (segment (start 126.492 86.36) (end 126.492 82.804) (width 0.25) (layer F.Cu) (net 1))
 (segment (start 124.714 81.000506) (end 123.952 80.238506) (width 0.25) (layer F.Cu) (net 1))
 (segment (start 126.492 82.804) (end 124.714 81.026) (width 0.25) (layer F.Cu) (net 1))
 (segment (start 124.714 81.026) (end 124.714 81.000506) (width 0.25) (layer F.Cu) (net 1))
 (segment (start 123.952 77.216) (end 126.746 74.422) (width 0.25) (layer F.Cu) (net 1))
 (segment (start 123.952 80.238506) (end 123.952 77.216) (width 0.25) (layer F.Cu) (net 1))
 (segment (start 134.112 78.74) (end 136.398 76.454) (width 0.25) (layer F.Cu) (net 2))
 (segment (start 139.446 75.522) (end 139.446 74.422) (width 0.25) (layer F.Cu) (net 2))
 (segment (start 138.514 76.454) (end 139.446 75.522) (width 0.25) (layer F.Cu) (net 2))
 (segment (start 136.398 76.454) (end 138.514 76.454) (width 0.25) (layer F.Cu) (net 2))
 (segment (start 131.572 78.74) (end 133.35 76.962) (width 0.25) (layer F.Cu) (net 4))
 (segment (start 134.366 76.962) (end 136.906 74.422) (width 0.25) (layer F.Cu) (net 4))
 (segment (start 133.35 76.962) (end 134.366 76.962) (width 0.25) (layer F.Cu) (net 4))
 (segment (start 129.032 78.74) (end 131.318 76.454) (width 0.25) (layer F.Cu) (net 6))
 (segment (start 131.318 76.454) (end 133.604 76.454) (width 0.25) (layer F.Cu) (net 6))
 (segment (start 134.366 75.692) (end 134.366 74.422) (width 0.25) (layer F.Cu) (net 6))
 (segment (start 133.604 76.454) (end 134.366 75.692) (width 0.25) (layer F.Cu) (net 6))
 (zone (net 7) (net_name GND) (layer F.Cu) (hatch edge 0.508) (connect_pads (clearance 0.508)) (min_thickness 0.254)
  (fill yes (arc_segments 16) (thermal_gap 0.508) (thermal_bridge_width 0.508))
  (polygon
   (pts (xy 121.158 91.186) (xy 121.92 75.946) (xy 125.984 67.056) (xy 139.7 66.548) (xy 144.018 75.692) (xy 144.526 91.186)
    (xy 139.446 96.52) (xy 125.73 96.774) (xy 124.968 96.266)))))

